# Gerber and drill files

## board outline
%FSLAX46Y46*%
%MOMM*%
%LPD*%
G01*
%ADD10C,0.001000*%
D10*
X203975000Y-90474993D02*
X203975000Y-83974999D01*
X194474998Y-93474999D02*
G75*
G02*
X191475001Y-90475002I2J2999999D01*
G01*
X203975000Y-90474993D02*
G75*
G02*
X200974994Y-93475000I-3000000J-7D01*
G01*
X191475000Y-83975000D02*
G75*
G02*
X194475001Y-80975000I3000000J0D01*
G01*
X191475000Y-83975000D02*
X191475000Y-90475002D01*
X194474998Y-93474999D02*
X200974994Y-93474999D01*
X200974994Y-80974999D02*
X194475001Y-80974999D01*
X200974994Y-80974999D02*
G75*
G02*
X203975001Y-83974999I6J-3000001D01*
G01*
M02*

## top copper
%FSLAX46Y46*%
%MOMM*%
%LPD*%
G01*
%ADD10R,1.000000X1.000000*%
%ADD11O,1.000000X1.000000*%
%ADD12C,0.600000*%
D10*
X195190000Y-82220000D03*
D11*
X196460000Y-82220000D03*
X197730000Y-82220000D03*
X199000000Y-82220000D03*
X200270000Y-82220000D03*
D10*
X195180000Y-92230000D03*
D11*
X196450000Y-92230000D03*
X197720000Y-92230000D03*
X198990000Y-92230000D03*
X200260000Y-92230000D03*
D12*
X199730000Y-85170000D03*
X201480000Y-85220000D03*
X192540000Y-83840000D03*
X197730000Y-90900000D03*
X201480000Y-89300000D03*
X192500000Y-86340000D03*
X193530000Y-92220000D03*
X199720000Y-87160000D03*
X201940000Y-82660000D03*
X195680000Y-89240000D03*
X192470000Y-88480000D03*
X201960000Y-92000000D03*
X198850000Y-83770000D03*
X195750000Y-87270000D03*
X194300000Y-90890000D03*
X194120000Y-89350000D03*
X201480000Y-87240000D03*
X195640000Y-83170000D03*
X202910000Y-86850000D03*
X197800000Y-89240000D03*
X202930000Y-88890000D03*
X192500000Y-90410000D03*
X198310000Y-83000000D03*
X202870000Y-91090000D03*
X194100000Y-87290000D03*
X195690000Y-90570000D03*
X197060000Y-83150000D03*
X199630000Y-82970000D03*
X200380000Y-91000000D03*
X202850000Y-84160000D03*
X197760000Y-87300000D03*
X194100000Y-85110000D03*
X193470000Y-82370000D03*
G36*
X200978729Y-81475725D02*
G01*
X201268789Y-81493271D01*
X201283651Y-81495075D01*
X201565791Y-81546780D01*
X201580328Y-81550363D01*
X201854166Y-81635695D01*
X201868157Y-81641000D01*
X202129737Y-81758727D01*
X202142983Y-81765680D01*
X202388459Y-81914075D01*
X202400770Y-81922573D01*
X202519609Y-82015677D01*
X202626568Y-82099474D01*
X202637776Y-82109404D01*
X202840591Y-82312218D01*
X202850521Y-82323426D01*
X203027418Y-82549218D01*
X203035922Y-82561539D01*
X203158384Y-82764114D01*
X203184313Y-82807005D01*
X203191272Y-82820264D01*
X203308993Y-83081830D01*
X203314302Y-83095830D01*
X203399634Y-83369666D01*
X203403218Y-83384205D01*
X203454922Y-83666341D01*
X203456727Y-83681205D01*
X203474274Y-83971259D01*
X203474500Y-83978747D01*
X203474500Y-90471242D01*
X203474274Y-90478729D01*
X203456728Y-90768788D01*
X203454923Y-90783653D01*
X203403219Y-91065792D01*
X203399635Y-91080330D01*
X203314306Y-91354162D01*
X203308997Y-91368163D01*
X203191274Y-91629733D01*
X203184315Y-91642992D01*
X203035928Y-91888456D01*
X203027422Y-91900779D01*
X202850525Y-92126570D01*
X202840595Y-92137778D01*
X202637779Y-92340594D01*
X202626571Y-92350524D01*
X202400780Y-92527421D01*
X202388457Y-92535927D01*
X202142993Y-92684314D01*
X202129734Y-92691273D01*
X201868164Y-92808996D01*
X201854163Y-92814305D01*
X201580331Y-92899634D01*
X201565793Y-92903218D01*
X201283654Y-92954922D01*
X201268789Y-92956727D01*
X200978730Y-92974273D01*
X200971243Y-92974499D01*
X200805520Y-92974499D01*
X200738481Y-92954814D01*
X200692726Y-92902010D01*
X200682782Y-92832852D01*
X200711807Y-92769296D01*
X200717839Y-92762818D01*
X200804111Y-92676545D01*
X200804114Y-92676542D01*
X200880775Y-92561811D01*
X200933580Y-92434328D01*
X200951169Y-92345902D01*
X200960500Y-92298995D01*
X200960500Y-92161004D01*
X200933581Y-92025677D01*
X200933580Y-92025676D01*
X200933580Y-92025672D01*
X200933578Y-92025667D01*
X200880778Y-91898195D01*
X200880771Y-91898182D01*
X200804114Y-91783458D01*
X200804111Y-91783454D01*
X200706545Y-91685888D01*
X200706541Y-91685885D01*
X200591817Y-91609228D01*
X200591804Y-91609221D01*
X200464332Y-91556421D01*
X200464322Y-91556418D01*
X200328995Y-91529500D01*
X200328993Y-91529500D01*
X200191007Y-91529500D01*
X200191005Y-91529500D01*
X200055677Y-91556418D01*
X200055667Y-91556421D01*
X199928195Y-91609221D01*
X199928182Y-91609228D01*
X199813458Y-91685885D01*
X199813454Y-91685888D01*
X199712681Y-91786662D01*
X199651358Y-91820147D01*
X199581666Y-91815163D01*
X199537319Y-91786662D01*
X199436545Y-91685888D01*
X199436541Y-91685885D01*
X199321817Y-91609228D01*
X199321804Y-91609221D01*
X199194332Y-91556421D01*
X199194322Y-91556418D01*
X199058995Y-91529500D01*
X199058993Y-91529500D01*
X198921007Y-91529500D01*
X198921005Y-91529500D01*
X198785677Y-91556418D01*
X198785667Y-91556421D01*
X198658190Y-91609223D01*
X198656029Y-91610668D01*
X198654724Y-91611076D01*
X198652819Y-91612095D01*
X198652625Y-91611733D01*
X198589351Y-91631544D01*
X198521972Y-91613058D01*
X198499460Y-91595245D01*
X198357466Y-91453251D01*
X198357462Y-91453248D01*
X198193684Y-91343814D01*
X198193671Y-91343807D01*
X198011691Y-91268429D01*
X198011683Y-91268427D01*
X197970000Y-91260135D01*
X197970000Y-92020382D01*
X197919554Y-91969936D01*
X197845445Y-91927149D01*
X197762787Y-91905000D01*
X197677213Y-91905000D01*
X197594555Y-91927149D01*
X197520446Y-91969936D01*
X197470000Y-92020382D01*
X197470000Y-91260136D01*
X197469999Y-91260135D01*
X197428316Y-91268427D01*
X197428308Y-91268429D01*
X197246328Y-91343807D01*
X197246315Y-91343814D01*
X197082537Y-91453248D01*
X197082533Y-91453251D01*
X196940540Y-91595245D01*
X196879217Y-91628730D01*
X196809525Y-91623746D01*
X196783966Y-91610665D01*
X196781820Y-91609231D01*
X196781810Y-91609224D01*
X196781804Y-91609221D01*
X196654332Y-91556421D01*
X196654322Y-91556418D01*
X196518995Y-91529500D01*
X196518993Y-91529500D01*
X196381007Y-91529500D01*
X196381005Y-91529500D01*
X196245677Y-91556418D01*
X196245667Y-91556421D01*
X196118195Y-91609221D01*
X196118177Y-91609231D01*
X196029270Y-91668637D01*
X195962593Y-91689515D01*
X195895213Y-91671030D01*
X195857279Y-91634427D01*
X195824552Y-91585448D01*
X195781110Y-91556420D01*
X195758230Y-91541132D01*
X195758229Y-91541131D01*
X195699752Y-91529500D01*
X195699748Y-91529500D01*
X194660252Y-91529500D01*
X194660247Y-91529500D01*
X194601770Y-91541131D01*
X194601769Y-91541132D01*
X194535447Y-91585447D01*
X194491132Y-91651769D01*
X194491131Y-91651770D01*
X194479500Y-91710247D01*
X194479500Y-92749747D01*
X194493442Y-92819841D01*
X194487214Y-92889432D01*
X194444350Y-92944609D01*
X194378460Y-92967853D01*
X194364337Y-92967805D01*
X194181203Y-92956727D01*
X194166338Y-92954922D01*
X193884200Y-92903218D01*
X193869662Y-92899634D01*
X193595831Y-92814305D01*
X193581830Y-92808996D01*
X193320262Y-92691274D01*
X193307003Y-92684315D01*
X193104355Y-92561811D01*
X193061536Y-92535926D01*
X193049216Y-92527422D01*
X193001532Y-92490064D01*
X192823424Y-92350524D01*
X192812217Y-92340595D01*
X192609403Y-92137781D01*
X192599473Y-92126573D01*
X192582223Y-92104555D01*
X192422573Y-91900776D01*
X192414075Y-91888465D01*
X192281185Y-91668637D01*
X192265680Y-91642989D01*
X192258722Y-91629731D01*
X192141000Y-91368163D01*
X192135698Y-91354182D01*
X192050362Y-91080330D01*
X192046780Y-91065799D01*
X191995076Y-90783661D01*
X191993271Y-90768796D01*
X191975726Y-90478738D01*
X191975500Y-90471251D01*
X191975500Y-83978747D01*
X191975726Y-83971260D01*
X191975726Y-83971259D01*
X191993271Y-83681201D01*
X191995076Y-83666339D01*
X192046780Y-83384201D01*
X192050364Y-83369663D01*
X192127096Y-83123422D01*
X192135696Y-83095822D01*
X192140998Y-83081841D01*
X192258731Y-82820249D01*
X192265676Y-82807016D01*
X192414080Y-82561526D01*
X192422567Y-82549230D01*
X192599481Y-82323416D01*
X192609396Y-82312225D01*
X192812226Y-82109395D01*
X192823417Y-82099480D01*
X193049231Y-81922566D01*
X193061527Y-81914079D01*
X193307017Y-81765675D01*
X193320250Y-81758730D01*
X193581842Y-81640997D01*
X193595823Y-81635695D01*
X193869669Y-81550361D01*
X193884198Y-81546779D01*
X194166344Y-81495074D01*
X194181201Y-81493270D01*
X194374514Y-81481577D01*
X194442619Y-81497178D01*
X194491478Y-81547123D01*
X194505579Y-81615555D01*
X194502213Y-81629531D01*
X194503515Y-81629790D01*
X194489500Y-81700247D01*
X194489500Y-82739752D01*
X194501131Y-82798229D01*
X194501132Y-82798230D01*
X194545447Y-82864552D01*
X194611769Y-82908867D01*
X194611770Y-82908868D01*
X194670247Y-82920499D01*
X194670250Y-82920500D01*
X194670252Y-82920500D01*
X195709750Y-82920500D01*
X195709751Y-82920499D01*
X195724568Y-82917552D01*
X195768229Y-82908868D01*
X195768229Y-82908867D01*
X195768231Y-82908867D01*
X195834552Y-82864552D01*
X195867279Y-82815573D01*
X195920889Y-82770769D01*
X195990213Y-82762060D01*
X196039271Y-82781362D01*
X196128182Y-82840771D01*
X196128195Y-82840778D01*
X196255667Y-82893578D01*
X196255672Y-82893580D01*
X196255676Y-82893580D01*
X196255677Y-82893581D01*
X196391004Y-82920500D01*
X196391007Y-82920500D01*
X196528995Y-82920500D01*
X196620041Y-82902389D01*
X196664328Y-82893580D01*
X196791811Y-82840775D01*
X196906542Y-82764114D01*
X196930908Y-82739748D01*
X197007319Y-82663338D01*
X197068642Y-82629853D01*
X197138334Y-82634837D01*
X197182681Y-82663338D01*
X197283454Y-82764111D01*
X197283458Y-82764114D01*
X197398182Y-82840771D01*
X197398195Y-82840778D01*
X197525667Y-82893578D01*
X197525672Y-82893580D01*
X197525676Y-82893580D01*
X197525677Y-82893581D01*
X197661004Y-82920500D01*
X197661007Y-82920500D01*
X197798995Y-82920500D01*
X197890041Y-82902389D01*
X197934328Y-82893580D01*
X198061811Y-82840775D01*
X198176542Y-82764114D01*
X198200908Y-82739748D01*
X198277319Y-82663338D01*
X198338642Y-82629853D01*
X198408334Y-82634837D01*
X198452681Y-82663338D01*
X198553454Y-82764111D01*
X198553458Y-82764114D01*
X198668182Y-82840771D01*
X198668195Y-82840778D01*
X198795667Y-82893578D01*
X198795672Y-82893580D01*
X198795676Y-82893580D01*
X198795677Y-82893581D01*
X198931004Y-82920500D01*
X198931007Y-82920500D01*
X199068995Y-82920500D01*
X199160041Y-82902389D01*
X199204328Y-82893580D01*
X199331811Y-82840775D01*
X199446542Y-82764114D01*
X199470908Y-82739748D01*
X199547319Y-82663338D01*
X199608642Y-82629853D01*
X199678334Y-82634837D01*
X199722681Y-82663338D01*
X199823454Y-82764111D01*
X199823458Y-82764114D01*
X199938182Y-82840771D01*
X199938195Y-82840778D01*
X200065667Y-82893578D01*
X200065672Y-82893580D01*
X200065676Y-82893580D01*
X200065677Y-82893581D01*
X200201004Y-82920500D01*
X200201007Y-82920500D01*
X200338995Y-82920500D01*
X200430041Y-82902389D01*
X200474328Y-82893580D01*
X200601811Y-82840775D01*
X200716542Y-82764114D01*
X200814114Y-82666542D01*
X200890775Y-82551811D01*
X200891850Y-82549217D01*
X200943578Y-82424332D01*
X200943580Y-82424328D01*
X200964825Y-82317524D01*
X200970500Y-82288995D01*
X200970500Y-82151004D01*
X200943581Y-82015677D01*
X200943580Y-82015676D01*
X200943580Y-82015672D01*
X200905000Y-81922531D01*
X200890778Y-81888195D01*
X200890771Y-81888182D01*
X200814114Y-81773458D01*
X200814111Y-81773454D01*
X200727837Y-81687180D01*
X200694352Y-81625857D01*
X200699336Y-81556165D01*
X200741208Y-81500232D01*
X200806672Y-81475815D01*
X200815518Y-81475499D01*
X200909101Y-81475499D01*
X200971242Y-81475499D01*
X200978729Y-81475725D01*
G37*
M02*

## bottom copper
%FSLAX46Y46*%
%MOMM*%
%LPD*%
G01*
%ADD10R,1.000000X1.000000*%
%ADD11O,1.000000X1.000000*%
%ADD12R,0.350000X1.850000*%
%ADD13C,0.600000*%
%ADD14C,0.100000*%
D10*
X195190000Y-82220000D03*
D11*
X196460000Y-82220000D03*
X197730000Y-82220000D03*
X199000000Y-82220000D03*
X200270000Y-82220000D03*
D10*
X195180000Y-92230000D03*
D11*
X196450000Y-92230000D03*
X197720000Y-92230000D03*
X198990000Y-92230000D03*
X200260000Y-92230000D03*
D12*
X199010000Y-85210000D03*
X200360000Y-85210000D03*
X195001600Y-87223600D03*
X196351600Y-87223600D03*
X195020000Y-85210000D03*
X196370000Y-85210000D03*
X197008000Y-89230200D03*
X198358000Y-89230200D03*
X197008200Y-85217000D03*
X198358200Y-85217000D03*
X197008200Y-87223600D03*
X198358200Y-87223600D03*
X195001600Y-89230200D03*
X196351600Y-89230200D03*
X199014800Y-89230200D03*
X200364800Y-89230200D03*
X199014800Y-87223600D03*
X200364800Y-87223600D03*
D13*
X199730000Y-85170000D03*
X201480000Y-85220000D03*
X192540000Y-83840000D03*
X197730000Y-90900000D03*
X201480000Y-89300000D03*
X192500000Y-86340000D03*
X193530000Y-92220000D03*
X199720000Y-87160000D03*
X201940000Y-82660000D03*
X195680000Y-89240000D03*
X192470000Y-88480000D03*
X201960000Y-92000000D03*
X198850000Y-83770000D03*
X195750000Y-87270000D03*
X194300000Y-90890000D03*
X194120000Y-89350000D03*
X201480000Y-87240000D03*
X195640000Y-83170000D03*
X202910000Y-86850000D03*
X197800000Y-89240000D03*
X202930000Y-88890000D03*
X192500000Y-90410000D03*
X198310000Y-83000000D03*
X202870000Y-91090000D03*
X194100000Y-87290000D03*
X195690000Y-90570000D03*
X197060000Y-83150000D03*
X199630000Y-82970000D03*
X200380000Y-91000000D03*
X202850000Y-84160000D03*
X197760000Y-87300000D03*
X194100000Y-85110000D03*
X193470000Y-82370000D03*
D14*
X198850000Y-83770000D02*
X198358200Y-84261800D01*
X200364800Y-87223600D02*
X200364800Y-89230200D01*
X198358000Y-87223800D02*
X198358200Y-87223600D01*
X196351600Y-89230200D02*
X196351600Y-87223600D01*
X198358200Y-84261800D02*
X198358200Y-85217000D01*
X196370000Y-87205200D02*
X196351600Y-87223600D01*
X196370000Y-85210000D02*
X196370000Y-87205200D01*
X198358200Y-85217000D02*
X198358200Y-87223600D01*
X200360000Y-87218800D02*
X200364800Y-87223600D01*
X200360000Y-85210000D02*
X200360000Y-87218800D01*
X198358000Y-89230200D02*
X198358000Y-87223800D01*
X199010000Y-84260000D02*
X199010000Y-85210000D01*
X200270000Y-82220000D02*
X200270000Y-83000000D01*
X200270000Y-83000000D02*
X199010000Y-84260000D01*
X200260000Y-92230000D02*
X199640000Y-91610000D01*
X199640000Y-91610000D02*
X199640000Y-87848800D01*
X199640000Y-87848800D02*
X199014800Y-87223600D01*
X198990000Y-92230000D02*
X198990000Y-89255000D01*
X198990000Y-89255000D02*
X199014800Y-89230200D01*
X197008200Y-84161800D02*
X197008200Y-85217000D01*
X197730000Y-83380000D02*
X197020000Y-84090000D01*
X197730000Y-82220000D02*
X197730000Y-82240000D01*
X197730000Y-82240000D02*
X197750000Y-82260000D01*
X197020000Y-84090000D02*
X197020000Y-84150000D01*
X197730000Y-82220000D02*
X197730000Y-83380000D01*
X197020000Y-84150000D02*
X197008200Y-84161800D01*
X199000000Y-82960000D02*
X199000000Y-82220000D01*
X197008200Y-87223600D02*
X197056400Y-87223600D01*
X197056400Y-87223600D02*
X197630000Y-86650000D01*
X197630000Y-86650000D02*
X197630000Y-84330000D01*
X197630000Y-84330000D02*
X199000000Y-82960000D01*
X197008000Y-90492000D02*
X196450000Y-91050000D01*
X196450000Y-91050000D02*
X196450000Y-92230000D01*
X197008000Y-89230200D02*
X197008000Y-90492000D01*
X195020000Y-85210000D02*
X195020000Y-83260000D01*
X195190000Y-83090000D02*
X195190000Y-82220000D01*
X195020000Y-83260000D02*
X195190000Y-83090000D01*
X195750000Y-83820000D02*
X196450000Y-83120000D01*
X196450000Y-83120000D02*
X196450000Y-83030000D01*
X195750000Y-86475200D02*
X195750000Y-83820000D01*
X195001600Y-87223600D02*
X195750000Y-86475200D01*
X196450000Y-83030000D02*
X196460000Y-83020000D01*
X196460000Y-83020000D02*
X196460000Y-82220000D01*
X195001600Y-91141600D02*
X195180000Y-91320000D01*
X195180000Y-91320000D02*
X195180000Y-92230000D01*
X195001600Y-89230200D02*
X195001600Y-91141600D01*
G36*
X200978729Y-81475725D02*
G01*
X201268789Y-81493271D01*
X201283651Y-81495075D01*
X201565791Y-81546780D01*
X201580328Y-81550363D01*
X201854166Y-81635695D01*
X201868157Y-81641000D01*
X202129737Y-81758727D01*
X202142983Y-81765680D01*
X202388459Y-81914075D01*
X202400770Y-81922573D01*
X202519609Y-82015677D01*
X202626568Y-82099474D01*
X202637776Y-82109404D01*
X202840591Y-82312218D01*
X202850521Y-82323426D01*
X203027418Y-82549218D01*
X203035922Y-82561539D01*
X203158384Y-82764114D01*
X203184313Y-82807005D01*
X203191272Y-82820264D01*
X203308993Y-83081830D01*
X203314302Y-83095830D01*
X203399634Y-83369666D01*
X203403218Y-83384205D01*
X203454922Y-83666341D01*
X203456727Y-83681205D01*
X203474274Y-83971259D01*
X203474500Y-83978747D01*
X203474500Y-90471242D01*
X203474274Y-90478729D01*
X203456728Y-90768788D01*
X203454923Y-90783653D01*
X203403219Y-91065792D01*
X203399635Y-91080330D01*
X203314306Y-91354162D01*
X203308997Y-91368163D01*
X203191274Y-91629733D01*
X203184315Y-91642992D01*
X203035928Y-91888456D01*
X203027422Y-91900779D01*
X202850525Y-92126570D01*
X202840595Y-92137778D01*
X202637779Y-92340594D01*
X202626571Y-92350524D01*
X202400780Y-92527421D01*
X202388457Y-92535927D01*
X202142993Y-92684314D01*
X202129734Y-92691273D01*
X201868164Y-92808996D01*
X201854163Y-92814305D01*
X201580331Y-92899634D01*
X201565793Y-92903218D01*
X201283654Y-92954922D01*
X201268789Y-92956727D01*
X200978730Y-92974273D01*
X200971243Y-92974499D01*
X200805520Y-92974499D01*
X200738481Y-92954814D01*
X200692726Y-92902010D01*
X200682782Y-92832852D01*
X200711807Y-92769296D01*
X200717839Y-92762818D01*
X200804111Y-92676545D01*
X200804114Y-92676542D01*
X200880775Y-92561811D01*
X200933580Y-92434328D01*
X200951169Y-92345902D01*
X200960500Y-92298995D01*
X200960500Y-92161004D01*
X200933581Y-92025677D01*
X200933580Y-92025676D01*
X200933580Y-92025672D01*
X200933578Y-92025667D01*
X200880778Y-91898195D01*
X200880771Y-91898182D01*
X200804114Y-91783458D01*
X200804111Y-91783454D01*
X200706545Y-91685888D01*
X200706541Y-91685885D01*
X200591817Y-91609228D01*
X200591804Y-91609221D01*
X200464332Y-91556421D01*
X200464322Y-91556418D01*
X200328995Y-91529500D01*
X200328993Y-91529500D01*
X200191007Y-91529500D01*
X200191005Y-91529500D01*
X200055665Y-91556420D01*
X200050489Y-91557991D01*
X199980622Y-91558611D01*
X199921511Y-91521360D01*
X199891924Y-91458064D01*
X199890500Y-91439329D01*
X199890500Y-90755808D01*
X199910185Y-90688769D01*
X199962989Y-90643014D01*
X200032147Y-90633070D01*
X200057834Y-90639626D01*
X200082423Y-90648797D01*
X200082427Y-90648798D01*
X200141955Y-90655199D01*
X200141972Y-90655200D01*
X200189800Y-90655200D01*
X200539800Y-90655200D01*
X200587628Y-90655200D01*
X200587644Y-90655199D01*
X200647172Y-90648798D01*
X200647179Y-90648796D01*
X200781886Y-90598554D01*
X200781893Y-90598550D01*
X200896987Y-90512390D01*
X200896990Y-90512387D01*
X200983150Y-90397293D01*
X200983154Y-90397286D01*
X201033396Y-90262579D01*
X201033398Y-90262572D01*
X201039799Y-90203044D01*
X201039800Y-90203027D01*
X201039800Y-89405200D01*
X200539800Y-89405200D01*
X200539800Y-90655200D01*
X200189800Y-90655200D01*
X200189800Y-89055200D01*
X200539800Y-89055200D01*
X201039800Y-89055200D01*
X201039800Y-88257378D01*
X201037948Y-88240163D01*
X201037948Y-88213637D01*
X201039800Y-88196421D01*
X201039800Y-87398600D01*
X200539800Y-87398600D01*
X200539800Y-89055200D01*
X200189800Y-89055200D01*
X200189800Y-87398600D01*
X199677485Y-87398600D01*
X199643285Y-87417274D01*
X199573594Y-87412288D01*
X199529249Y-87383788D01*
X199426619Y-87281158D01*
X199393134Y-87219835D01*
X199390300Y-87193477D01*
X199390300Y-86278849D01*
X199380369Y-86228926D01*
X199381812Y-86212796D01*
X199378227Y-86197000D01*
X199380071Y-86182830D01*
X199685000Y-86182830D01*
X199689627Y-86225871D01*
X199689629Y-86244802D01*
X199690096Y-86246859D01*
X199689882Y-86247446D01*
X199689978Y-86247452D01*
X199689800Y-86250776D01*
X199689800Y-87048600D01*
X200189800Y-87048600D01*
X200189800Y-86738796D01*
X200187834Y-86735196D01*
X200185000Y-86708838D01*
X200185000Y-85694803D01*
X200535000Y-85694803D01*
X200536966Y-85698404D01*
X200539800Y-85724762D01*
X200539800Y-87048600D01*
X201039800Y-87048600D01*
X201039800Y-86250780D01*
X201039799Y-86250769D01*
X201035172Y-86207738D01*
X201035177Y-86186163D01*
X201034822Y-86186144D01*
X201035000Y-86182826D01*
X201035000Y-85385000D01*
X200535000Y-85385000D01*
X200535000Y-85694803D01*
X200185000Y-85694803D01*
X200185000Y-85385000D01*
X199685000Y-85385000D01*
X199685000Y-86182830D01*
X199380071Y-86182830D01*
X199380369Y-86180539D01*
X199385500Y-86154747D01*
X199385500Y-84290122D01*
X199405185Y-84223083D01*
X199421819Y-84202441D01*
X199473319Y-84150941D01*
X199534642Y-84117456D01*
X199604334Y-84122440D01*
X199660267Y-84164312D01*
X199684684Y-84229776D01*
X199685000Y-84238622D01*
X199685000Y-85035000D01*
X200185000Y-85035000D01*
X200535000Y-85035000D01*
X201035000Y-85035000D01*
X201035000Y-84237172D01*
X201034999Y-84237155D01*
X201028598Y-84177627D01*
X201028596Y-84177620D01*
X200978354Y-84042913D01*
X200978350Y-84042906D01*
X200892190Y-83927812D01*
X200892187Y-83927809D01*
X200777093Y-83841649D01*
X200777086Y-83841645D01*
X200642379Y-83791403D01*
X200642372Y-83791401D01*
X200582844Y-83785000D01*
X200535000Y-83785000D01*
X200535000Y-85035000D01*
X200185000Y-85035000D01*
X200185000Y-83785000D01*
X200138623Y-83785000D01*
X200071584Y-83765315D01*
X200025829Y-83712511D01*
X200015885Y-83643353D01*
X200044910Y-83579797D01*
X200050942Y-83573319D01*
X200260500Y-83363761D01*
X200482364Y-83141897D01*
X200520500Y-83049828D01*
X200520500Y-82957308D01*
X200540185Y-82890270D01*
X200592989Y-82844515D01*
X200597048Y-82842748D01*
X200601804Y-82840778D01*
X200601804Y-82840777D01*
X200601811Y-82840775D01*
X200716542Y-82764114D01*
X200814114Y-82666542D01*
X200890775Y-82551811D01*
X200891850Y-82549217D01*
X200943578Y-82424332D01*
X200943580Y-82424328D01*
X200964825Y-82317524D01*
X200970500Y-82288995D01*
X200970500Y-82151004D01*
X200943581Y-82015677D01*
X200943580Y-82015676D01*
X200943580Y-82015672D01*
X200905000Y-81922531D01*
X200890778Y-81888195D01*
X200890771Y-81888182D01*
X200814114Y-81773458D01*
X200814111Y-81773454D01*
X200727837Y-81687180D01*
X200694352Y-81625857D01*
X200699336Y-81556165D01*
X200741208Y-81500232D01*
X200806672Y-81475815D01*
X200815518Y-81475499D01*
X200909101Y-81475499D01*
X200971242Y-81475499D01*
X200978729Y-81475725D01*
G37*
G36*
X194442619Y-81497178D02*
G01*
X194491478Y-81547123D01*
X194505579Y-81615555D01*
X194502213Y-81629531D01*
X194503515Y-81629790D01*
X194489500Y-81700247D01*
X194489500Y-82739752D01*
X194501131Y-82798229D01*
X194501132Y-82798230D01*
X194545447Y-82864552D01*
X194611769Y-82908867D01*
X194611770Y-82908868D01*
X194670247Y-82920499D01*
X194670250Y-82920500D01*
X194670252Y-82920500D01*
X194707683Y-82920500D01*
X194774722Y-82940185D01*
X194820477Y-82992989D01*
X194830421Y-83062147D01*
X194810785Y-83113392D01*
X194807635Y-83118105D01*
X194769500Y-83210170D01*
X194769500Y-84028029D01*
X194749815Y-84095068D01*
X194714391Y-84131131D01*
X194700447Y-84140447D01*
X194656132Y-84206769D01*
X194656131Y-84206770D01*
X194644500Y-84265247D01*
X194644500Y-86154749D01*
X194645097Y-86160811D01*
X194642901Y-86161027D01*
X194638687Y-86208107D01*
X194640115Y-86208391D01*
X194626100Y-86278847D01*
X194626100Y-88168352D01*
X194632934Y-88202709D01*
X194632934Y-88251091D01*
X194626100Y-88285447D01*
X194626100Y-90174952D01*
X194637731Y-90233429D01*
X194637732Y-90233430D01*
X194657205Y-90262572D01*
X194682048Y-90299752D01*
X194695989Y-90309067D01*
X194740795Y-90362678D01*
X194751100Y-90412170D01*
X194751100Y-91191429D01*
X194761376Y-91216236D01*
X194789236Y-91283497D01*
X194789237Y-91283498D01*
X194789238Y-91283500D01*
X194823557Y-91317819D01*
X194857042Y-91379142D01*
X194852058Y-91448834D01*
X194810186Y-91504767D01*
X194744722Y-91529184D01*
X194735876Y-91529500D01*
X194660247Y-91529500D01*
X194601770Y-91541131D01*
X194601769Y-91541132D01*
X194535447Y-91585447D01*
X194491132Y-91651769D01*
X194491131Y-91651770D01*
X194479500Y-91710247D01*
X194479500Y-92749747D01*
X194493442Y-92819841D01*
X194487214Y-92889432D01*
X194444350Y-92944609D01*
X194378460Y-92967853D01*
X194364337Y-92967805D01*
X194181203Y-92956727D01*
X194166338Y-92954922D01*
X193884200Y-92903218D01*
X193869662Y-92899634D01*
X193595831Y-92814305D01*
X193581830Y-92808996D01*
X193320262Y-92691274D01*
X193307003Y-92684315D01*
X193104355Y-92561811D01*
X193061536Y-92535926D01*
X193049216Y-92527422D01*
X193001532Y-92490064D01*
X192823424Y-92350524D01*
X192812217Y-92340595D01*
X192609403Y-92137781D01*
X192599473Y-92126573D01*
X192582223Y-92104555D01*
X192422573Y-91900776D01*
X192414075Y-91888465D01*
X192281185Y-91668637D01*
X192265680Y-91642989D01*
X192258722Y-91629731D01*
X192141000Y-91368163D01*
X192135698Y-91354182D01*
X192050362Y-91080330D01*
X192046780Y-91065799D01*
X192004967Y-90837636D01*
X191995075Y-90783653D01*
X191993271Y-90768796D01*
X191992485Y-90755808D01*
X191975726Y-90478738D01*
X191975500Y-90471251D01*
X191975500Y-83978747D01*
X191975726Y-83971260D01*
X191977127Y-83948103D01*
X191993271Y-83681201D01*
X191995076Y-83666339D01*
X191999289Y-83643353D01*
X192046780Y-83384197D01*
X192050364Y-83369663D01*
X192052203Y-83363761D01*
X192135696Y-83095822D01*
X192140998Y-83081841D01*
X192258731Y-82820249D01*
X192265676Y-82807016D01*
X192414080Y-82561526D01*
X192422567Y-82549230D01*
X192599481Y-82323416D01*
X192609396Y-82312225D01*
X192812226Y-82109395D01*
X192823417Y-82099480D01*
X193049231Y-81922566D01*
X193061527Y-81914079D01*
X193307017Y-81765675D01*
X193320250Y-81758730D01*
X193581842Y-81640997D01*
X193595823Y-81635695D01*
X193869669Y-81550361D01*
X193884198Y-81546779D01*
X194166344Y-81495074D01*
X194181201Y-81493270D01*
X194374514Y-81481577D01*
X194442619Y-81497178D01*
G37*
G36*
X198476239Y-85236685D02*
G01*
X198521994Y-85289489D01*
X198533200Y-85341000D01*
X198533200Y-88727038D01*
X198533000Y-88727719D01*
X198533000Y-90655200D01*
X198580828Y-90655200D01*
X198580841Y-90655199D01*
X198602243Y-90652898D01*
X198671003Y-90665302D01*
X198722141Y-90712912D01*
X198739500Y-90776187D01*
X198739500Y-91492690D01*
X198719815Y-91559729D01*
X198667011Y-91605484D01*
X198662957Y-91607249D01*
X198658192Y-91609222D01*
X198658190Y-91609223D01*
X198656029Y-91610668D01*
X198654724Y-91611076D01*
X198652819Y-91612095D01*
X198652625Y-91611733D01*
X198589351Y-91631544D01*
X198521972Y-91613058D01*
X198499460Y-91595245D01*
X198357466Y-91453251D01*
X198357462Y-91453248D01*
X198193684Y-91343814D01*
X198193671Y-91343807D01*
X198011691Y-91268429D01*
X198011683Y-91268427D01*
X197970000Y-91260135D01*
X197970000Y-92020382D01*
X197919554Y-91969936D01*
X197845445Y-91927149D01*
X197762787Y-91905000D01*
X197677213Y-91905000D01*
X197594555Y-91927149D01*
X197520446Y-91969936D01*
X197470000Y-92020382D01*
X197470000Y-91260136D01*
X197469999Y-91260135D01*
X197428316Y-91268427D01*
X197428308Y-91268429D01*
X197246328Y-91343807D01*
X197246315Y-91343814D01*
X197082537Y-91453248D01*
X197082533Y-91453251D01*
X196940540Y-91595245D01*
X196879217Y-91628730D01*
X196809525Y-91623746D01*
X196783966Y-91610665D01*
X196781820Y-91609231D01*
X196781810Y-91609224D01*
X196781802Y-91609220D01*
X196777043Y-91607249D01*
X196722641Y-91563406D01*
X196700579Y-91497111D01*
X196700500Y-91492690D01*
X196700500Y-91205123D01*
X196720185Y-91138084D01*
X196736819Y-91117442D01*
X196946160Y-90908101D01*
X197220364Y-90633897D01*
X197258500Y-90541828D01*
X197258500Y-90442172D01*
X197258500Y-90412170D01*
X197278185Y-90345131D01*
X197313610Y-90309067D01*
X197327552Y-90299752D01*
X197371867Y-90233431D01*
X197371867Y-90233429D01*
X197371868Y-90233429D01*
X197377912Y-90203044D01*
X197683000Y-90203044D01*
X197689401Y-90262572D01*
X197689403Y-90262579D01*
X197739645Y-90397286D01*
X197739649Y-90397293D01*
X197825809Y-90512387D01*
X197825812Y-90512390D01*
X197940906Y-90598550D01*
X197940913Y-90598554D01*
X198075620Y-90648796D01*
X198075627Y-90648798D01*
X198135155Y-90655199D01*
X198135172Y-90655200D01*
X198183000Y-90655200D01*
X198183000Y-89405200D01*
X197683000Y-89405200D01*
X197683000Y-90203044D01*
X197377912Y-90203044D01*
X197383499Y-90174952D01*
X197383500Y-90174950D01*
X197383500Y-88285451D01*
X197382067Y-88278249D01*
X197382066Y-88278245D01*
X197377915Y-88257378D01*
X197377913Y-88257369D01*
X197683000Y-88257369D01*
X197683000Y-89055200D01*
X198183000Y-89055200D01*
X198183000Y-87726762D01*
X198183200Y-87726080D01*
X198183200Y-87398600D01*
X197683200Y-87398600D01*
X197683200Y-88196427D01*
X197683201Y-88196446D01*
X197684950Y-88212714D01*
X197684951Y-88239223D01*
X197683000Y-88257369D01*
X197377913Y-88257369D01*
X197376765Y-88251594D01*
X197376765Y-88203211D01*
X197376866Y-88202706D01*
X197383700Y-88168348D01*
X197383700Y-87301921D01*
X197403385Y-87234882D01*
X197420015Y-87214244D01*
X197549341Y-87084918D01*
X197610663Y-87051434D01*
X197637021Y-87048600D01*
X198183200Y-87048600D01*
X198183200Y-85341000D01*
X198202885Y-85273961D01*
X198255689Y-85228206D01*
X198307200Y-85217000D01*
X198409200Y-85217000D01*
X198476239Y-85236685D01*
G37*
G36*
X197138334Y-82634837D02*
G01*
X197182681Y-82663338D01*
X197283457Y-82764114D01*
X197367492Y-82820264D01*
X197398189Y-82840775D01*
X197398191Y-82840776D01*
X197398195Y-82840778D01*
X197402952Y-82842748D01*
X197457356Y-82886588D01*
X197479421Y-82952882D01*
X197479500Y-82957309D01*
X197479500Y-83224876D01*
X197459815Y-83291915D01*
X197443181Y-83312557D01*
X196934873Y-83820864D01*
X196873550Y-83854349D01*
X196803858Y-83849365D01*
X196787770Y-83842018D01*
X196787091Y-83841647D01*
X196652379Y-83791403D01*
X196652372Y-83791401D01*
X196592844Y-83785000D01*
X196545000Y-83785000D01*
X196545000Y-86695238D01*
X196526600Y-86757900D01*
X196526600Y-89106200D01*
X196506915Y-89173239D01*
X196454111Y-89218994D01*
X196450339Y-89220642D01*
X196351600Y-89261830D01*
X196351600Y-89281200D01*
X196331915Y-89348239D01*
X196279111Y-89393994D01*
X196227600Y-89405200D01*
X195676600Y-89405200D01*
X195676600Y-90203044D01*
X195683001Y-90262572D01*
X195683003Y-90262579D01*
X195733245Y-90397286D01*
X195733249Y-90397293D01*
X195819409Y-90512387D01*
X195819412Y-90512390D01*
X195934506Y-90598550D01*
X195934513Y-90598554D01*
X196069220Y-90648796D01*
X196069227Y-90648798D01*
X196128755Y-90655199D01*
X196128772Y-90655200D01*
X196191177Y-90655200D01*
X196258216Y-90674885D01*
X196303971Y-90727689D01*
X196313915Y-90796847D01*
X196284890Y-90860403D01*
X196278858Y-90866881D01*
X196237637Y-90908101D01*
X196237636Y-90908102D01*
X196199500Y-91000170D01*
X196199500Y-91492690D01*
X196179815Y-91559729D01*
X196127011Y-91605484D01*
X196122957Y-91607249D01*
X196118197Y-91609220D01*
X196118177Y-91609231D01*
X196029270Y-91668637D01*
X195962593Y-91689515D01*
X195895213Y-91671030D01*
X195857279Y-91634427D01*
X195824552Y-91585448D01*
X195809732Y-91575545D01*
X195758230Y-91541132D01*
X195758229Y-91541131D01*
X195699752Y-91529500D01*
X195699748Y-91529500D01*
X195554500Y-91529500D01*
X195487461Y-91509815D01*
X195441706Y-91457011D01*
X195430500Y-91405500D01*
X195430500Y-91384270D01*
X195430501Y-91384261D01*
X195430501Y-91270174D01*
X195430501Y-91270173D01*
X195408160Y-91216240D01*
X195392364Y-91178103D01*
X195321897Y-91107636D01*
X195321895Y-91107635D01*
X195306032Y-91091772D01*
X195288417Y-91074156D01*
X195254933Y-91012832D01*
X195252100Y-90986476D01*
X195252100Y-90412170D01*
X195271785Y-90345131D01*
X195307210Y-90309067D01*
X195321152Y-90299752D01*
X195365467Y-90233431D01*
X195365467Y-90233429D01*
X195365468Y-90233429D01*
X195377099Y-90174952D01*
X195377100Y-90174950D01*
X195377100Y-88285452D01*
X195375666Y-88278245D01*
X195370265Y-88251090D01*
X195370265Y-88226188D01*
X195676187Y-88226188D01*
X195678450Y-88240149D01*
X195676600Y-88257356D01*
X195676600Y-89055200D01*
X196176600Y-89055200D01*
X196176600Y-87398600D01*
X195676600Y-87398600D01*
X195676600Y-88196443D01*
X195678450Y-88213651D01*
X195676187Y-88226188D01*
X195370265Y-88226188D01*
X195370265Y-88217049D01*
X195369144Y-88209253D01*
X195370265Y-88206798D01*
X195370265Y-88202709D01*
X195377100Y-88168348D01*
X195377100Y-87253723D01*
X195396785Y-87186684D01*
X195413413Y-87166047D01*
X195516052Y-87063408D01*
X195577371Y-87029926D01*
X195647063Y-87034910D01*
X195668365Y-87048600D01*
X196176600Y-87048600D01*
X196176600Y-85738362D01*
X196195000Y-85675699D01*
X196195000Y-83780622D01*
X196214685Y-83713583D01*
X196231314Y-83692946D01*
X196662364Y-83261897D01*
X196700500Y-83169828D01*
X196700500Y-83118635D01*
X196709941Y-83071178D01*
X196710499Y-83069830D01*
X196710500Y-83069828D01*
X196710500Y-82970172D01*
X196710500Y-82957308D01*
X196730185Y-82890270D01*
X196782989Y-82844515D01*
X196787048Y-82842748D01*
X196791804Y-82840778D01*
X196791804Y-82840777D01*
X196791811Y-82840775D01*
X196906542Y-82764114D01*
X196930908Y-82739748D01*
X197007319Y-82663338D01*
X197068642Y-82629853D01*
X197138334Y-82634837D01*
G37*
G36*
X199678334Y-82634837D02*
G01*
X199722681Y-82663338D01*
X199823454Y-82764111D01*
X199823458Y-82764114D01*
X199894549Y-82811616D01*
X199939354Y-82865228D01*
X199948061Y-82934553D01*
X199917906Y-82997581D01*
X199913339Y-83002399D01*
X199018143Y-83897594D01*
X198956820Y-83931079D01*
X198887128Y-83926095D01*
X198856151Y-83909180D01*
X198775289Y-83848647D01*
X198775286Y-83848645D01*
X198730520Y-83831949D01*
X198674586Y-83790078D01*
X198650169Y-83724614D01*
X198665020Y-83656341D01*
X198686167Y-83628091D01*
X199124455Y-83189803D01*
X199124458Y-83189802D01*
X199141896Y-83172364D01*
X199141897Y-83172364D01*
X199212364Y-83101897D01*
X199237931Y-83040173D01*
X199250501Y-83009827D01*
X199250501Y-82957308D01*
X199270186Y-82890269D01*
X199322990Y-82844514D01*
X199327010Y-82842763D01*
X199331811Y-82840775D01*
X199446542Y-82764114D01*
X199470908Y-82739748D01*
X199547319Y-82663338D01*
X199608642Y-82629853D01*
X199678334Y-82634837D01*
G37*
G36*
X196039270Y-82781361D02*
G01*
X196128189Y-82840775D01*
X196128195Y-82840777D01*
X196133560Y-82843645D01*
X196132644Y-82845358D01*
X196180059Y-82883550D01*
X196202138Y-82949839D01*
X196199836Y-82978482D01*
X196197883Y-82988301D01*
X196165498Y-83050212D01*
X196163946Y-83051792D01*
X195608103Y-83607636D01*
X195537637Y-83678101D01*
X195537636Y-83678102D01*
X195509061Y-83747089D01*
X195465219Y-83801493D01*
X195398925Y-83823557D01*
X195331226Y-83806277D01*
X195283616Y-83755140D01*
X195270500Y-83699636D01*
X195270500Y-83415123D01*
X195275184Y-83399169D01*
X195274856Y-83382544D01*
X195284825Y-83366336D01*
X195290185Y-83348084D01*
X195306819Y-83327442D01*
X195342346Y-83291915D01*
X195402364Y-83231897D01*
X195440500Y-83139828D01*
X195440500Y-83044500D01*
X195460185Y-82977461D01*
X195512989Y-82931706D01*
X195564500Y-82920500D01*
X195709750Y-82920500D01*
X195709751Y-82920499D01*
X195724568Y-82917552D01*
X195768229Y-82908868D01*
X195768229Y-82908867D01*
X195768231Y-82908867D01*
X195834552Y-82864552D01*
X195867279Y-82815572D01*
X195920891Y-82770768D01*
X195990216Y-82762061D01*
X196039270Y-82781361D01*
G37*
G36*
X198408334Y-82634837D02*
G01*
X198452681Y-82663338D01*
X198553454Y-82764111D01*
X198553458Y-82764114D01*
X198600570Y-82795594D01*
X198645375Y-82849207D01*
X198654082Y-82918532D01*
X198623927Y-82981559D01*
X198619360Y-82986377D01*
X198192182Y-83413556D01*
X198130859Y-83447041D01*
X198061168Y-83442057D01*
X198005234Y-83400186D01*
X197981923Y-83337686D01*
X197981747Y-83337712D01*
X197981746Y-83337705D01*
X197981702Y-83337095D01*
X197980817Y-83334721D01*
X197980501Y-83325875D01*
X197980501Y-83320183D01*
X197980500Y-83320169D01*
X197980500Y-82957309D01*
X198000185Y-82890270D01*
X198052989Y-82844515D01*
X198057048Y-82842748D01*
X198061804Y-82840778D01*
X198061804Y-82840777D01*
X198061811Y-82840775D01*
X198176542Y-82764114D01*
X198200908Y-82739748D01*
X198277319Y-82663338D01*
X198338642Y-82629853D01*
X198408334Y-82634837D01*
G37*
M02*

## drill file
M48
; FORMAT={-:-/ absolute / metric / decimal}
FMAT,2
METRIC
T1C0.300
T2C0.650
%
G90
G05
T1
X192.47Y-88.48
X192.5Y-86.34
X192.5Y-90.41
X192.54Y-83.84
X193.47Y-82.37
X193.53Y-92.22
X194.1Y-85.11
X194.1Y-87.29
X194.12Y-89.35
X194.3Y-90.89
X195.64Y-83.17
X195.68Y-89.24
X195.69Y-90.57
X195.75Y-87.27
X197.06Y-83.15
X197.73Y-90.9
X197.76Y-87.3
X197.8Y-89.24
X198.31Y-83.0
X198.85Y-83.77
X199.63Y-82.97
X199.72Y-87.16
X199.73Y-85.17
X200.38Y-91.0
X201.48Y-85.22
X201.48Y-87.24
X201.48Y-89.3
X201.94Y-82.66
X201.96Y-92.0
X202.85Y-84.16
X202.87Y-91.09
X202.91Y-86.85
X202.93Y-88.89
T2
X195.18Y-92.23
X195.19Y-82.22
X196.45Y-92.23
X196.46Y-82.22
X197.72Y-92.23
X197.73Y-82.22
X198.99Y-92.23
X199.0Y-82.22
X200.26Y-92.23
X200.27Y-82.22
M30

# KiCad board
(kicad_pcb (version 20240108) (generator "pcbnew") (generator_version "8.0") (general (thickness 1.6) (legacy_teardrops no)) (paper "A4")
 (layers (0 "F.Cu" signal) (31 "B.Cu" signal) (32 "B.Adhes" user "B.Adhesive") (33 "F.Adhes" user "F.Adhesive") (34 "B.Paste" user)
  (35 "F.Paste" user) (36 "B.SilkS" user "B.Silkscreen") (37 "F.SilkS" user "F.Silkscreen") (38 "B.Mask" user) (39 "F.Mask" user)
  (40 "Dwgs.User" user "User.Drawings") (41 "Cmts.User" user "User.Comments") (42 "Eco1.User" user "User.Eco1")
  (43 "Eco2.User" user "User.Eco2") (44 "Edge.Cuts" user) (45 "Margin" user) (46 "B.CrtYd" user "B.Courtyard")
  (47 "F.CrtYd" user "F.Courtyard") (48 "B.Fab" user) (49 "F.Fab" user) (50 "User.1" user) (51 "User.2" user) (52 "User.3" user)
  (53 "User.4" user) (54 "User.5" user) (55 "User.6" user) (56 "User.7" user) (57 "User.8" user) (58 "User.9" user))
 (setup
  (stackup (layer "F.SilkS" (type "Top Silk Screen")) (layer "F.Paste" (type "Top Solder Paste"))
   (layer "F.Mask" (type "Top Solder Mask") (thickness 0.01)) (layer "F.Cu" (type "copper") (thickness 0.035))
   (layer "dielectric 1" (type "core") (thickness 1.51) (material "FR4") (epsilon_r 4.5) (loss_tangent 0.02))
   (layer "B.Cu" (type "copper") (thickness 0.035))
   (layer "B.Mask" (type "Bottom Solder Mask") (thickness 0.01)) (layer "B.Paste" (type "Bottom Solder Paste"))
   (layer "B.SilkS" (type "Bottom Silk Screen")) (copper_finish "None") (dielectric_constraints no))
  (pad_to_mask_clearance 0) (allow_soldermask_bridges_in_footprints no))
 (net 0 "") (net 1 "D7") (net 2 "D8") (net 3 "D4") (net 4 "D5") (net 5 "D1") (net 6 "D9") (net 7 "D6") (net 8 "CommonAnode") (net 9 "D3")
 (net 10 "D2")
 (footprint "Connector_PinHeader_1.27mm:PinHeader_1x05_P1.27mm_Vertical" (layer "F.Cu") (at 195.19 82.22 90)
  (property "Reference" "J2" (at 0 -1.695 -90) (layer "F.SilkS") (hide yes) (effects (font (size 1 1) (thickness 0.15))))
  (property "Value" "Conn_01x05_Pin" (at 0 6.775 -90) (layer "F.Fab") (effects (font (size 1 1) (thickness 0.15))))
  (pad "1" thru_hole rect (at 0 0 90) (size 1 1) (drill 0.65) (layers "*.Cu" "*.Mask") (remove_unused_layers no) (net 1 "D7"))
  (pad "2" thru_hole oval (at 0 1.27 90) (size 1 1) (drill 0.65) (layers "*.Cu" "*.Mask") (remove_unused_layers no) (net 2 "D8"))
  (pad "3" thru_hole oval (at 0 2.54 90) (size 1 1) (drill 0.65) (layers "*.Cu" "*.Mask") (remove_unused_layers no) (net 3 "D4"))
  (pad "4" thru_hole oval (at 0 3.81 90) (size 1 1) (drill 0.65) (layers "*.Cu" "*.Mask") (remove_unused_layers no) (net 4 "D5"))
  (pad "5" thru_hole oval (at 0 5.08 90) (size 1 1) (drill 0.65) (layers "*.Cu" "*.Mask") (remove_unused_layers no) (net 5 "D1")))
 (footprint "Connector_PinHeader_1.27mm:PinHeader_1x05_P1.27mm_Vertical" (layer "F.Cu") (at 195.18 92.23 90)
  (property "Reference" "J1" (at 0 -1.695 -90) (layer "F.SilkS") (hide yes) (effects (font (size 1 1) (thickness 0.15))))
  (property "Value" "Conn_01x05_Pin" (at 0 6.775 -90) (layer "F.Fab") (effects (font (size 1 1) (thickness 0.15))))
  (pad "1" thru_hole rect (at 0 0 90) (size 1 1) (drill 0.65) (layers "*.Cu" "*.Mask") (remove_unused_layers no) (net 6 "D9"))
  (pad "2" thru_hole oval (at 0 1.27 90) (size 1 1) (drill 0.65) (layers "*.Cu" "*.Mask") (remove_unused_layers no) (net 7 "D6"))
  (pad "3" thru_hole oval (at 0 2.54 90) (size 1 1) (drill 0.65) (layers "*.Cu" "*.Mask") (remove_unused_layers no) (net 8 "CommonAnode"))
  (pad "4" thru_hole oval (at 0 3.81 90) (size 1 1) (drill 0.65) (layers "*.Cu" "*.Mask") (remove_unused_layers no) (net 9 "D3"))
  (pad "5" thru_hole oval (at 0 5.08 90) (size 1 1) (drill 0.65) (layers "*.Cu" "*.Mask") (remove_unused_layers no) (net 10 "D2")))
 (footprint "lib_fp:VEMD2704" (layer "B.Cu") (at 199.69 85.21 -90)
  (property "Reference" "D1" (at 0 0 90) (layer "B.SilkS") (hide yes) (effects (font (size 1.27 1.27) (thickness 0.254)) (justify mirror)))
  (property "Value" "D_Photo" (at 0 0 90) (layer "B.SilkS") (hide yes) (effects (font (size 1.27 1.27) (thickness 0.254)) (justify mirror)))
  (pad "1" smd rect (at 0 0.68 180) (size 0.35 1.85) (layers "B.Cu" "B.Paste" "B.Mask") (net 5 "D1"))
  (pad "2" smd rect (at 0 -0.67 180) (size 0.35 1.85) (layers "B.Cu" "B.Paste" "B.Mask") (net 8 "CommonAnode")))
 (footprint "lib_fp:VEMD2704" (layer "B.Cu") (at 195.6816 87.2236 -90)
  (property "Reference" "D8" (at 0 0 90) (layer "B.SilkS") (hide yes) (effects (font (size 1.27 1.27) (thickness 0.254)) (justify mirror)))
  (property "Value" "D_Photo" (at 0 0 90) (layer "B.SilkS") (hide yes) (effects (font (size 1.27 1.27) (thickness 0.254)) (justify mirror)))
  (pad "1" smd rect (at 0 0.68 180) (size 0.35 1.85) (layers "B.Cu" "B.Paste" "B.Mask") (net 2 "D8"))
  (pad "2" smd rect (at 0 -0.67 180) (size 0.35 1.85) (layers "B.Cu" "B.Paste" "B.Mask") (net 8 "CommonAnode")))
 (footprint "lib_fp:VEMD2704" (layer "B.Cu") (at 195.7 85.21 -90)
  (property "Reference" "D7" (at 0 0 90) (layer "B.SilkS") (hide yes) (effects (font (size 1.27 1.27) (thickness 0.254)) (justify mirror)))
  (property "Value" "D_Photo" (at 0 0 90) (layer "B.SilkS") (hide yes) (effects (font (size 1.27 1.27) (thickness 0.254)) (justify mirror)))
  (pad "1" smd rect (at 0 0.68 180) (size 0.35 1.85) (layers "B.Cu" "B.Paste" "B.Mask") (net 1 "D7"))
  (pad "2" smd rect (at 0 -0.67 180) (size 0.35 1.85) (layers "B.Cu" "B.Paste" "B.Mask") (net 8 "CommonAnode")))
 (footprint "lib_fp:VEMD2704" (layer "B.Cu") (at 197.688 89.2302 -90)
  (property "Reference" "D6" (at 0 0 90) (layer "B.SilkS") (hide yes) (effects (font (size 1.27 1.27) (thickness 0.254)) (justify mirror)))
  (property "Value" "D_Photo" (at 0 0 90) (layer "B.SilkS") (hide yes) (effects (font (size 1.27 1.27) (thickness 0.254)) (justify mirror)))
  (pad "1" smd rect (at 0 0.68 180) (size 0.35 1.85) (layers "B.Cu" "B.Paste" "B.Mask") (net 7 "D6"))
  (pad "2" smd rect (at 0 -0.67 180) (size 0.35 1.85) (layers "B.Cu" "B.Paste" "B.Mask") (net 8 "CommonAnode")))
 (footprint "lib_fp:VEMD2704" (layer "B.Cu") (at 197.6882 85.217 -90)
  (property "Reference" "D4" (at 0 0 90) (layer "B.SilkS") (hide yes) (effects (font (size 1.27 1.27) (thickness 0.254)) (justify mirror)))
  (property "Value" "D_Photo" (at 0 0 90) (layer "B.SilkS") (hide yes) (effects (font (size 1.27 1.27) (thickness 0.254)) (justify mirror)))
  (pad "1" smd rect (at 0 0.68 180) (size 0.35 1.85) (layers "B.Cu" "B.Paste" "B.Mask") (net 3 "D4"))
  (pad "2" smd rect (at 0 -0.67 180) (size 0.35 1.85) (layers "B.Cu" "B.Paste" "B.Mask") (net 8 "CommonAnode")))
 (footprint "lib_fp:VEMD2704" (layer "B.Cu") (at 197.6882 87.2236 -90)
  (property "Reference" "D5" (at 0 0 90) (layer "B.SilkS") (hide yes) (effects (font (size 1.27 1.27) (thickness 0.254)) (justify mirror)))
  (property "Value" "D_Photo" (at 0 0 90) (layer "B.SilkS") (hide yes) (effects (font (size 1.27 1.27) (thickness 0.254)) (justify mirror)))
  (pad "1" smd rect (at 0 0.68 180) (size 0.35 1.85) (layers "B.Cu" "B.Paste" "B.Mask") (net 4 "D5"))
  (pad "2" smd rect (at 0 -0.67 180) (size 0.35 1.85) (layers "B.Cu" "B.Paste" "B.Mask") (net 8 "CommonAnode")))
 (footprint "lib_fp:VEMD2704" (layer "B.Cu") (at 195.6816 89.2302 -90)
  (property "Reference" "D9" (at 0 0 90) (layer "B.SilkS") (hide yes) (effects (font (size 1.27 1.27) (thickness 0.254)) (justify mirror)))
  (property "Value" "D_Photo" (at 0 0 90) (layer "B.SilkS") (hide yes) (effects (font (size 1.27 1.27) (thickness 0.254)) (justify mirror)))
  (pad "1" smd rect (at 0 0.68 180) (size 0.35 1.85) (layers "B.Cu" "B.Paste" "B.Mask") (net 6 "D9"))
  (pad "2" smd rect (at 0 -0.67 180) (size 0.35 1.85) (layers "B.Cu" "B.Paste" "B.Mask") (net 8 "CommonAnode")))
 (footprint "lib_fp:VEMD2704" (layer "B.Cu") (at 199.6948 89.2302 -90)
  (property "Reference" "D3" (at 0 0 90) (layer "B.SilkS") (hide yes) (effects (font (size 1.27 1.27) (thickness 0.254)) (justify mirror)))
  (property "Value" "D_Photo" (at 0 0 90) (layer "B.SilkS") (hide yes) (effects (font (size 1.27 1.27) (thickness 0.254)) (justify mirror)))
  (pad "1" smd rect (at 0 0.68 180) (size 0.35 1.85) (layers "B.Cu" "B.Paste" "B.Mask") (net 9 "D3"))
  (pad "2" smd rect (at 0 -0.67 180) (size 0.35 1.85) (layers "B.Cu" "B.Paste" "B.Mask") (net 8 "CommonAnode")))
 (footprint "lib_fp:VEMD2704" (layer "B.Cu") (at 199.6948 87.2236 -90)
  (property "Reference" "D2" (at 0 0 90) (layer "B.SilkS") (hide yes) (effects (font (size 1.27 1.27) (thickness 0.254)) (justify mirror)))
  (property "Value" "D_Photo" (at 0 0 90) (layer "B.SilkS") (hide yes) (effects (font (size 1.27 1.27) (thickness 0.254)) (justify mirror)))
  (pad "1" smd rect (at 0 0.68 180) (size 0.35 1.85) (layers "B.Cu" "B.Paste" "B.Mask") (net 10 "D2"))
  (pad "2" smd rect (at 0 -0.67 180) (size 0.35 1.85) (layers "B.Cu" "B.Paste" "B.Mask") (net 8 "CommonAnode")))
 (gr_line (start 203.975 90.474993) (end 203.975 83.974999) (stroke (width 0.001) (type default)) (layer "Edge.Cuts"))
 (gr_arc (start 194.474998 93.474999) (mid 192.353679 92.59632) (end 191.475 90.475002) (stroke (width 0.001) (type default))
  (layer "Edge.Cuts"))
 (gr_arc (start 203.975 90.474993) (mid 203.096319 92.596318) (end 200.974994 93.474999) (stroke (width 0.001) (type default))
  (layer "Edge.Cuts"))
 (gr_arc (start 191.475 83.975) (mid 192.35368 81.853679) (end 194.475001 80.974999) (stroke (width 0.001) (type default))
  (layer "Edge.Cuts"))
 (gr_line (start 191.475 83.975) (end 191.475 90.475002) (stroke (width 0.001) (type default)) (layer "Edge.Cuts"))
 (gr_line (start 194.474998 93.474999) (end 200.974994 93.474999) (stroke (width 0.001) (type default)) (layer "Edge.Cuts"))
 (gr_line (start 200.974994 80.974999) (end 194.475001 80.974999) (stroke (width 0.001) (type default)) (layer "Edge.Cuts"))
 (gr_arc (start 200.974994 80.974999) (mid 203.096314 81.853679) (end 203.975 83.974999) (stroke (width 0.001) (type default))
  (layer "Edge.Cuts"))
 (via (at 199.73 85.17) (size 0.6) (drill 0.3) (layers "F.Cu" "B.Cu") (free yes) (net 8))
 (via (at 201.48 85.22) (size 0.6) (drill 0.3) (layers "F.Cu" "B.Cu") (free yes) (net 8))
 (via (at 192.54 83.84) (size 0.6) (drill 0.3) (layers "F.Cu" "B.Cu") (free yes) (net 8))
 (via (at 197.73 90.9) (size 0.6) (drill 0.3) (layers "F.Cu" "B.Cu") (free yes) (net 8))
 (via (at 201.48 89.3) (size 0.6) (drill 0.3) (layers "F.Cu" "B.Cu") (free yes) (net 8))
 (via (at 192.5 86.34) (size 0.6) (drill 0.3) (layers "F.Cu" "B.Cu") (free yes) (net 8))
 (via (at 193.53 92.22) (size 0.6) (drill 0.3) (layers "F.Cu" "B.Cu") (free yes) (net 8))
 (via (at 199.72 87.16) (size 0.6) (drill 0.3) (layers "F.Cu" "B.Cu") (free yes) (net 8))
 (via (at 201.94 82.66) (size 0.6) (drill 0.3) (layers "F.Cu" "B.Cu") (free yes) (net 8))
 (via (at 195.68 89.24) (size 0.6) (drill 0.3) (layers "F.Cu" "B.Cu") (free yes) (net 8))
 (via (at 192.47 88.48) (size 0.6) (drill 0.3) (layers "F.Cu" "B.Cu") (free yes) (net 8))
 (via (at 201.96 92) (size 0.6) (drill 0.3) (layers "F.Cu" "B.Cu") (free yes) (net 8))
 (via (at 198.85 83.77) (size 0.6) (drill 0.3) (layers "F.Cu" "B.Cu") (free yes) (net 8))
 (via (at 195.75 87.27) (size 0.6) (drill 0.3) (layers "F.Cu" "B.Cu") (free yes) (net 8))
 (via (at 194.3 90.89) (size 0.6) (drill 0.3) (layers "F.Cu" "B.Cu") (free yes) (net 8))
 (via (at 194.12 89.35) (size 0.6) (drill 0.3) (layers "F.Cu" "B.Cu") (free yes) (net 8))
 (via (at 201.48 87.24) (size 0.6) (drill 0.3) (layers "F.Cu" "B.Cu") (free yes) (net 8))
 (via (at 195.64 83.17) (size 0.6) (drill 0.3) (layers "F.Cu" "B.Cu") (free yes) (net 8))
 (via (at 202.91 86.85) (size 0.6) (drill 0.3) (layers "F.Cu" "B.Cu") (free yes) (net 8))
 (via (at 197.8 89.24) (size 0.6) (drill 0.3) (layers "F.Cu" "B.Cu") (free yes) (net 8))
 (via (at 202.93 88.89) (size 0.6) (drill 0.3) (layers "F.Cu" "B.Cu") (free yes) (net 8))
 (via (at 192.5 90.41) (size 0.6) (drill 0.3) (layers "F.Cu" "B.Cu") (free yes) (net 8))
 (via (at 198.31 83) (size 0.6) (drill 0.3) (layers "F.Cu" "B.Cu") (free yes) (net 8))
 (via (at 202.87 91.09) (size 0.6) (drill 0.3) (layers "F.Cu" "B.Cu") (free yes) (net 8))
 (via (at 194.1 87.29) (size 0.6) (drill 0.3) (layers "F.Cu" "B.Cu") (free yes) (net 8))
 (via (at 195.69 90.57) (size 0.6) (drill 0.3) (layers "F.Cu" "B.Cu") (free yes) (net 8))
 (via (at 197.06 83.15) (size 0.6) (drill 0.3) (layers "F.Cu" "B.Cu") (free yes) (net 8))
 (via (at 199.63 82.97) (size 0.6) (drill 0.3) (layers "F.Cu" "B.Cu") (free yes) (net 8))
 (via (at 200.38 91) (size 0.6) (drill 0.3) (layers "F.Cu" "B.Cu") (free yes) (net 8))
 (via (at 202.85 84.16) (size 0.6) (drill 0.3) (layers "F.Cu" "B.Cu") (free yes) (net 8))
 (via (at 197.76 87.3) (size 0.6) (drill 0.3) (layers "F.Cu" "B.Cu") (free yes) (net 8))
 (via (at 194.1 85.11) (size 0.6) (drill 0.3) (layers "F.Cu" "B.Cu") (free yes) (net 8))
 (via (at 193.47 82.37) (size 0.6) (drill 0.3) (layers "F.Cu" "B.Cu") (free yes) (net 8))
 (segment (start 198.85 83.77) (end 198.3582 84.2618) (width 0.1) (layer "B.Cu") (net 8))
 (segment (start 200.3648 87.2236) (end 200.3648 89.2302) (width 0.1) (layer "B.Cu") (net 8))
 (segment (start 198.358 87.2238) (end 198.3582 87.2236) (width 0.1) (layer "B.Cu") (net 8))
 (segment (start 196.3516 89.2302) (end 196.3516 87.2236) (width 0.1) (layer "B.Cu") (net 8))
 (segment (start 198.3582 84.2618) (end 198.3582 85.217) (width 0.1) (layer "B.Cu") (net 8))
 (segment (start 196.37 87.2052) (end 196.3516 87.2236) (width 0.1) (layer "B.Cu") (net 8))
 (segment (start 196.37 85.21) (end 196.37 87.2052) (width 0.1) (layer "B.Cu") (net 8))
 (segment (start 198.3582 85.217) (end 198.3582 87.2236) (width 0.1) (layer "B.Cu") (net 8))
 (segment (start 200.36 87.2188) (end 200.3648 87.2236) (width 0.1) (layer "B.Cu") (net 8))
 (segment (start 200.36 85.21) (end 200.36 87.2188) (width 0.1) (layer "B.Cu") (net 8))
 (segment (start 198.358 89.2302) (end 198.358 87.2238) (width 0.1) (layer "B.Cu") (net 8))
 (segment (start 199.01 84.26) (end 199.01 85.21) (width 0.1) (layer "B.Cu") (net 5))
 (segment (start 200.27 82.22) (end 200.27 83) (width 0.1) (layer "B.Cu") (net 5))
 (segment (start 200.27 83) (end 199.01 84.26) (width 0.1) (layer "B.Cu") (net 5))
 (segment (start 200.26 92.23) (end 199.64 91.61) (width 0.1) (layer "B.Cu") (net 10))
 (segment (start 199.64 91.61) (end 199.64 87.8488) (width 0.1) (layer "B.Cu") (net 10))
 (segment (start 199.64 87.8488) (end 199.0148 87.2236) (width 0.1) (layer "B.Cu") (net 10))
 (segment (start 198.99 92.23) (end 198.99 89.255) (width 0.1) (layer "B.Cu") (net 9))
 (segment (start 198.99 89.255) (end 199.0148 89.2302) (width 0.1) (layer "B.Cu") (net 9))
 (segment (start 197.0082 84.1618) (end 197.0082 85.217) (width 0.1) (layer "B.Cu") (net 3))
 (segment (start 197.73 83.38) (end 197.02 84.09) (width 0.1) (layer "B.Cu") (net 3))
 (segment (start 197.73 82.22) (end 197.73 82.24) (width 0.1) (layer "B.Cu") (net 3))
 (segment (start 197.73 82.24) (end 197.75 82.26) (width 0.1) (layer "B.Cu") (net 3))
 (segment (start 197.02 84.09) (end 197.02 84.15) (width 0.1) (layer "B.Cu") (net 3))
 (segment (start 197.73 82.22) (end 197.73 83.38) (width 0.1) (layer "B.Cu") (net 3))
 (segment (start 197.02 84.15) (end 197.0082 84.1618) (width 0.1) (layer "B.Cu") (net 3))
 (segment (start 199 82.96) (end 199 82.22) (width 0.1) (layer "B.Cu") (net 4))
 (segment (start 197.0082 87.2236) (end 197.0564 87.2236) (width 0.1) (layer "B.Cu") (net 4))
 (segment (start 197.0564 87.2236) (end 197.63 86.65) (width 0.1) (layer "B.Cu") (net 4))
 (segment (start 197.63 86.65) (end 197.63 84.33) (width 0.1) (layer "B.Cu") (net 4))
 (segment (start 197.63 84.33) (end 199 82.96) (width 0.1) (layer "B.Cu") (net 4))
 (segment (start 197.008 90.492) (end 196.45 91.05) (width 0.1) (layer "B.Cu") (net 7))
 (segment (start 196.45 91.05) (end 196.45 92.23) (width 0.1) (layer "B.Cu") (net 7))
 (segment (start 197.008 89.2302) (end 197.008 90.492) (width 0.1) (layer "B.Cu") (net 7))
 (segment (start 195.02 85.21) (end 195.02 83.26) (width 0.1) (layer "B.Cu") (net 1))
 (segment (start 195.19 83.09) (end 195.19 82.22) (width 0.1) (layer "B.Cu") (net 1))
 (segment (start 195.02 83.26) (end 195.19 83.09) (width 0.1) (layer "B.Cu") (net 1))
 (segment (start 195.75 83.82) (end 196.45 83.12) (width 0.1) (layer "B.Cu") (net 2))
 (segment (start 196.45 83.12) (end 196.45 83.03) (width 0.1) (layer "B.Cu") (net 2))
 (segment (start 195.75 86.4752) (end 195.75 83.82) (width 0.1) (layer "B.Cu") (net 2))
 (segment (start 195.0016 87.2236) (end 195.75 86.4752) (width 0.1) (layer "B.Cu") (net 2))
 (segment (start 196.45 83.03) (end 196.46 83.02) (width 0.1) (layer "B.Cu") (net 2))
 (segment (start 196.46 83.02) (end 196.46 82.22) (width 0.1) (layer "B.Cu") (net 2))
 (segment (start 195.0016 91.1416) (end 195.18 91.32) (width 0.1) (layer "B.Cu") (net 6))
 (segment (start 195.18 91.32) (end 195.18 92.23) (width 0.1) (layer "B.Cu") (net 6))
 (segment (start 195.0016 89.2302) (end 195.0016 91.1416) (width 0.1) (layer "B.Cu") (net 6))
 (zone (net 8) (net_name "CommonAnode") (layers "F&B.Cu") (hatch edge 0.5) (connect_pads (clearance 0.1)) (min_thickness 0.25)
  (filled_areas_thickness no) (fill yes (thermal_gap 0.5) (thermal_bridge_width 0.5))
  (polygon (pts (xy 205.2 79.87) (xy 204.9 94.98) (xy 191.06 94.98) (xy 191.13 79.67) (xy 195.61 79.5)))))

